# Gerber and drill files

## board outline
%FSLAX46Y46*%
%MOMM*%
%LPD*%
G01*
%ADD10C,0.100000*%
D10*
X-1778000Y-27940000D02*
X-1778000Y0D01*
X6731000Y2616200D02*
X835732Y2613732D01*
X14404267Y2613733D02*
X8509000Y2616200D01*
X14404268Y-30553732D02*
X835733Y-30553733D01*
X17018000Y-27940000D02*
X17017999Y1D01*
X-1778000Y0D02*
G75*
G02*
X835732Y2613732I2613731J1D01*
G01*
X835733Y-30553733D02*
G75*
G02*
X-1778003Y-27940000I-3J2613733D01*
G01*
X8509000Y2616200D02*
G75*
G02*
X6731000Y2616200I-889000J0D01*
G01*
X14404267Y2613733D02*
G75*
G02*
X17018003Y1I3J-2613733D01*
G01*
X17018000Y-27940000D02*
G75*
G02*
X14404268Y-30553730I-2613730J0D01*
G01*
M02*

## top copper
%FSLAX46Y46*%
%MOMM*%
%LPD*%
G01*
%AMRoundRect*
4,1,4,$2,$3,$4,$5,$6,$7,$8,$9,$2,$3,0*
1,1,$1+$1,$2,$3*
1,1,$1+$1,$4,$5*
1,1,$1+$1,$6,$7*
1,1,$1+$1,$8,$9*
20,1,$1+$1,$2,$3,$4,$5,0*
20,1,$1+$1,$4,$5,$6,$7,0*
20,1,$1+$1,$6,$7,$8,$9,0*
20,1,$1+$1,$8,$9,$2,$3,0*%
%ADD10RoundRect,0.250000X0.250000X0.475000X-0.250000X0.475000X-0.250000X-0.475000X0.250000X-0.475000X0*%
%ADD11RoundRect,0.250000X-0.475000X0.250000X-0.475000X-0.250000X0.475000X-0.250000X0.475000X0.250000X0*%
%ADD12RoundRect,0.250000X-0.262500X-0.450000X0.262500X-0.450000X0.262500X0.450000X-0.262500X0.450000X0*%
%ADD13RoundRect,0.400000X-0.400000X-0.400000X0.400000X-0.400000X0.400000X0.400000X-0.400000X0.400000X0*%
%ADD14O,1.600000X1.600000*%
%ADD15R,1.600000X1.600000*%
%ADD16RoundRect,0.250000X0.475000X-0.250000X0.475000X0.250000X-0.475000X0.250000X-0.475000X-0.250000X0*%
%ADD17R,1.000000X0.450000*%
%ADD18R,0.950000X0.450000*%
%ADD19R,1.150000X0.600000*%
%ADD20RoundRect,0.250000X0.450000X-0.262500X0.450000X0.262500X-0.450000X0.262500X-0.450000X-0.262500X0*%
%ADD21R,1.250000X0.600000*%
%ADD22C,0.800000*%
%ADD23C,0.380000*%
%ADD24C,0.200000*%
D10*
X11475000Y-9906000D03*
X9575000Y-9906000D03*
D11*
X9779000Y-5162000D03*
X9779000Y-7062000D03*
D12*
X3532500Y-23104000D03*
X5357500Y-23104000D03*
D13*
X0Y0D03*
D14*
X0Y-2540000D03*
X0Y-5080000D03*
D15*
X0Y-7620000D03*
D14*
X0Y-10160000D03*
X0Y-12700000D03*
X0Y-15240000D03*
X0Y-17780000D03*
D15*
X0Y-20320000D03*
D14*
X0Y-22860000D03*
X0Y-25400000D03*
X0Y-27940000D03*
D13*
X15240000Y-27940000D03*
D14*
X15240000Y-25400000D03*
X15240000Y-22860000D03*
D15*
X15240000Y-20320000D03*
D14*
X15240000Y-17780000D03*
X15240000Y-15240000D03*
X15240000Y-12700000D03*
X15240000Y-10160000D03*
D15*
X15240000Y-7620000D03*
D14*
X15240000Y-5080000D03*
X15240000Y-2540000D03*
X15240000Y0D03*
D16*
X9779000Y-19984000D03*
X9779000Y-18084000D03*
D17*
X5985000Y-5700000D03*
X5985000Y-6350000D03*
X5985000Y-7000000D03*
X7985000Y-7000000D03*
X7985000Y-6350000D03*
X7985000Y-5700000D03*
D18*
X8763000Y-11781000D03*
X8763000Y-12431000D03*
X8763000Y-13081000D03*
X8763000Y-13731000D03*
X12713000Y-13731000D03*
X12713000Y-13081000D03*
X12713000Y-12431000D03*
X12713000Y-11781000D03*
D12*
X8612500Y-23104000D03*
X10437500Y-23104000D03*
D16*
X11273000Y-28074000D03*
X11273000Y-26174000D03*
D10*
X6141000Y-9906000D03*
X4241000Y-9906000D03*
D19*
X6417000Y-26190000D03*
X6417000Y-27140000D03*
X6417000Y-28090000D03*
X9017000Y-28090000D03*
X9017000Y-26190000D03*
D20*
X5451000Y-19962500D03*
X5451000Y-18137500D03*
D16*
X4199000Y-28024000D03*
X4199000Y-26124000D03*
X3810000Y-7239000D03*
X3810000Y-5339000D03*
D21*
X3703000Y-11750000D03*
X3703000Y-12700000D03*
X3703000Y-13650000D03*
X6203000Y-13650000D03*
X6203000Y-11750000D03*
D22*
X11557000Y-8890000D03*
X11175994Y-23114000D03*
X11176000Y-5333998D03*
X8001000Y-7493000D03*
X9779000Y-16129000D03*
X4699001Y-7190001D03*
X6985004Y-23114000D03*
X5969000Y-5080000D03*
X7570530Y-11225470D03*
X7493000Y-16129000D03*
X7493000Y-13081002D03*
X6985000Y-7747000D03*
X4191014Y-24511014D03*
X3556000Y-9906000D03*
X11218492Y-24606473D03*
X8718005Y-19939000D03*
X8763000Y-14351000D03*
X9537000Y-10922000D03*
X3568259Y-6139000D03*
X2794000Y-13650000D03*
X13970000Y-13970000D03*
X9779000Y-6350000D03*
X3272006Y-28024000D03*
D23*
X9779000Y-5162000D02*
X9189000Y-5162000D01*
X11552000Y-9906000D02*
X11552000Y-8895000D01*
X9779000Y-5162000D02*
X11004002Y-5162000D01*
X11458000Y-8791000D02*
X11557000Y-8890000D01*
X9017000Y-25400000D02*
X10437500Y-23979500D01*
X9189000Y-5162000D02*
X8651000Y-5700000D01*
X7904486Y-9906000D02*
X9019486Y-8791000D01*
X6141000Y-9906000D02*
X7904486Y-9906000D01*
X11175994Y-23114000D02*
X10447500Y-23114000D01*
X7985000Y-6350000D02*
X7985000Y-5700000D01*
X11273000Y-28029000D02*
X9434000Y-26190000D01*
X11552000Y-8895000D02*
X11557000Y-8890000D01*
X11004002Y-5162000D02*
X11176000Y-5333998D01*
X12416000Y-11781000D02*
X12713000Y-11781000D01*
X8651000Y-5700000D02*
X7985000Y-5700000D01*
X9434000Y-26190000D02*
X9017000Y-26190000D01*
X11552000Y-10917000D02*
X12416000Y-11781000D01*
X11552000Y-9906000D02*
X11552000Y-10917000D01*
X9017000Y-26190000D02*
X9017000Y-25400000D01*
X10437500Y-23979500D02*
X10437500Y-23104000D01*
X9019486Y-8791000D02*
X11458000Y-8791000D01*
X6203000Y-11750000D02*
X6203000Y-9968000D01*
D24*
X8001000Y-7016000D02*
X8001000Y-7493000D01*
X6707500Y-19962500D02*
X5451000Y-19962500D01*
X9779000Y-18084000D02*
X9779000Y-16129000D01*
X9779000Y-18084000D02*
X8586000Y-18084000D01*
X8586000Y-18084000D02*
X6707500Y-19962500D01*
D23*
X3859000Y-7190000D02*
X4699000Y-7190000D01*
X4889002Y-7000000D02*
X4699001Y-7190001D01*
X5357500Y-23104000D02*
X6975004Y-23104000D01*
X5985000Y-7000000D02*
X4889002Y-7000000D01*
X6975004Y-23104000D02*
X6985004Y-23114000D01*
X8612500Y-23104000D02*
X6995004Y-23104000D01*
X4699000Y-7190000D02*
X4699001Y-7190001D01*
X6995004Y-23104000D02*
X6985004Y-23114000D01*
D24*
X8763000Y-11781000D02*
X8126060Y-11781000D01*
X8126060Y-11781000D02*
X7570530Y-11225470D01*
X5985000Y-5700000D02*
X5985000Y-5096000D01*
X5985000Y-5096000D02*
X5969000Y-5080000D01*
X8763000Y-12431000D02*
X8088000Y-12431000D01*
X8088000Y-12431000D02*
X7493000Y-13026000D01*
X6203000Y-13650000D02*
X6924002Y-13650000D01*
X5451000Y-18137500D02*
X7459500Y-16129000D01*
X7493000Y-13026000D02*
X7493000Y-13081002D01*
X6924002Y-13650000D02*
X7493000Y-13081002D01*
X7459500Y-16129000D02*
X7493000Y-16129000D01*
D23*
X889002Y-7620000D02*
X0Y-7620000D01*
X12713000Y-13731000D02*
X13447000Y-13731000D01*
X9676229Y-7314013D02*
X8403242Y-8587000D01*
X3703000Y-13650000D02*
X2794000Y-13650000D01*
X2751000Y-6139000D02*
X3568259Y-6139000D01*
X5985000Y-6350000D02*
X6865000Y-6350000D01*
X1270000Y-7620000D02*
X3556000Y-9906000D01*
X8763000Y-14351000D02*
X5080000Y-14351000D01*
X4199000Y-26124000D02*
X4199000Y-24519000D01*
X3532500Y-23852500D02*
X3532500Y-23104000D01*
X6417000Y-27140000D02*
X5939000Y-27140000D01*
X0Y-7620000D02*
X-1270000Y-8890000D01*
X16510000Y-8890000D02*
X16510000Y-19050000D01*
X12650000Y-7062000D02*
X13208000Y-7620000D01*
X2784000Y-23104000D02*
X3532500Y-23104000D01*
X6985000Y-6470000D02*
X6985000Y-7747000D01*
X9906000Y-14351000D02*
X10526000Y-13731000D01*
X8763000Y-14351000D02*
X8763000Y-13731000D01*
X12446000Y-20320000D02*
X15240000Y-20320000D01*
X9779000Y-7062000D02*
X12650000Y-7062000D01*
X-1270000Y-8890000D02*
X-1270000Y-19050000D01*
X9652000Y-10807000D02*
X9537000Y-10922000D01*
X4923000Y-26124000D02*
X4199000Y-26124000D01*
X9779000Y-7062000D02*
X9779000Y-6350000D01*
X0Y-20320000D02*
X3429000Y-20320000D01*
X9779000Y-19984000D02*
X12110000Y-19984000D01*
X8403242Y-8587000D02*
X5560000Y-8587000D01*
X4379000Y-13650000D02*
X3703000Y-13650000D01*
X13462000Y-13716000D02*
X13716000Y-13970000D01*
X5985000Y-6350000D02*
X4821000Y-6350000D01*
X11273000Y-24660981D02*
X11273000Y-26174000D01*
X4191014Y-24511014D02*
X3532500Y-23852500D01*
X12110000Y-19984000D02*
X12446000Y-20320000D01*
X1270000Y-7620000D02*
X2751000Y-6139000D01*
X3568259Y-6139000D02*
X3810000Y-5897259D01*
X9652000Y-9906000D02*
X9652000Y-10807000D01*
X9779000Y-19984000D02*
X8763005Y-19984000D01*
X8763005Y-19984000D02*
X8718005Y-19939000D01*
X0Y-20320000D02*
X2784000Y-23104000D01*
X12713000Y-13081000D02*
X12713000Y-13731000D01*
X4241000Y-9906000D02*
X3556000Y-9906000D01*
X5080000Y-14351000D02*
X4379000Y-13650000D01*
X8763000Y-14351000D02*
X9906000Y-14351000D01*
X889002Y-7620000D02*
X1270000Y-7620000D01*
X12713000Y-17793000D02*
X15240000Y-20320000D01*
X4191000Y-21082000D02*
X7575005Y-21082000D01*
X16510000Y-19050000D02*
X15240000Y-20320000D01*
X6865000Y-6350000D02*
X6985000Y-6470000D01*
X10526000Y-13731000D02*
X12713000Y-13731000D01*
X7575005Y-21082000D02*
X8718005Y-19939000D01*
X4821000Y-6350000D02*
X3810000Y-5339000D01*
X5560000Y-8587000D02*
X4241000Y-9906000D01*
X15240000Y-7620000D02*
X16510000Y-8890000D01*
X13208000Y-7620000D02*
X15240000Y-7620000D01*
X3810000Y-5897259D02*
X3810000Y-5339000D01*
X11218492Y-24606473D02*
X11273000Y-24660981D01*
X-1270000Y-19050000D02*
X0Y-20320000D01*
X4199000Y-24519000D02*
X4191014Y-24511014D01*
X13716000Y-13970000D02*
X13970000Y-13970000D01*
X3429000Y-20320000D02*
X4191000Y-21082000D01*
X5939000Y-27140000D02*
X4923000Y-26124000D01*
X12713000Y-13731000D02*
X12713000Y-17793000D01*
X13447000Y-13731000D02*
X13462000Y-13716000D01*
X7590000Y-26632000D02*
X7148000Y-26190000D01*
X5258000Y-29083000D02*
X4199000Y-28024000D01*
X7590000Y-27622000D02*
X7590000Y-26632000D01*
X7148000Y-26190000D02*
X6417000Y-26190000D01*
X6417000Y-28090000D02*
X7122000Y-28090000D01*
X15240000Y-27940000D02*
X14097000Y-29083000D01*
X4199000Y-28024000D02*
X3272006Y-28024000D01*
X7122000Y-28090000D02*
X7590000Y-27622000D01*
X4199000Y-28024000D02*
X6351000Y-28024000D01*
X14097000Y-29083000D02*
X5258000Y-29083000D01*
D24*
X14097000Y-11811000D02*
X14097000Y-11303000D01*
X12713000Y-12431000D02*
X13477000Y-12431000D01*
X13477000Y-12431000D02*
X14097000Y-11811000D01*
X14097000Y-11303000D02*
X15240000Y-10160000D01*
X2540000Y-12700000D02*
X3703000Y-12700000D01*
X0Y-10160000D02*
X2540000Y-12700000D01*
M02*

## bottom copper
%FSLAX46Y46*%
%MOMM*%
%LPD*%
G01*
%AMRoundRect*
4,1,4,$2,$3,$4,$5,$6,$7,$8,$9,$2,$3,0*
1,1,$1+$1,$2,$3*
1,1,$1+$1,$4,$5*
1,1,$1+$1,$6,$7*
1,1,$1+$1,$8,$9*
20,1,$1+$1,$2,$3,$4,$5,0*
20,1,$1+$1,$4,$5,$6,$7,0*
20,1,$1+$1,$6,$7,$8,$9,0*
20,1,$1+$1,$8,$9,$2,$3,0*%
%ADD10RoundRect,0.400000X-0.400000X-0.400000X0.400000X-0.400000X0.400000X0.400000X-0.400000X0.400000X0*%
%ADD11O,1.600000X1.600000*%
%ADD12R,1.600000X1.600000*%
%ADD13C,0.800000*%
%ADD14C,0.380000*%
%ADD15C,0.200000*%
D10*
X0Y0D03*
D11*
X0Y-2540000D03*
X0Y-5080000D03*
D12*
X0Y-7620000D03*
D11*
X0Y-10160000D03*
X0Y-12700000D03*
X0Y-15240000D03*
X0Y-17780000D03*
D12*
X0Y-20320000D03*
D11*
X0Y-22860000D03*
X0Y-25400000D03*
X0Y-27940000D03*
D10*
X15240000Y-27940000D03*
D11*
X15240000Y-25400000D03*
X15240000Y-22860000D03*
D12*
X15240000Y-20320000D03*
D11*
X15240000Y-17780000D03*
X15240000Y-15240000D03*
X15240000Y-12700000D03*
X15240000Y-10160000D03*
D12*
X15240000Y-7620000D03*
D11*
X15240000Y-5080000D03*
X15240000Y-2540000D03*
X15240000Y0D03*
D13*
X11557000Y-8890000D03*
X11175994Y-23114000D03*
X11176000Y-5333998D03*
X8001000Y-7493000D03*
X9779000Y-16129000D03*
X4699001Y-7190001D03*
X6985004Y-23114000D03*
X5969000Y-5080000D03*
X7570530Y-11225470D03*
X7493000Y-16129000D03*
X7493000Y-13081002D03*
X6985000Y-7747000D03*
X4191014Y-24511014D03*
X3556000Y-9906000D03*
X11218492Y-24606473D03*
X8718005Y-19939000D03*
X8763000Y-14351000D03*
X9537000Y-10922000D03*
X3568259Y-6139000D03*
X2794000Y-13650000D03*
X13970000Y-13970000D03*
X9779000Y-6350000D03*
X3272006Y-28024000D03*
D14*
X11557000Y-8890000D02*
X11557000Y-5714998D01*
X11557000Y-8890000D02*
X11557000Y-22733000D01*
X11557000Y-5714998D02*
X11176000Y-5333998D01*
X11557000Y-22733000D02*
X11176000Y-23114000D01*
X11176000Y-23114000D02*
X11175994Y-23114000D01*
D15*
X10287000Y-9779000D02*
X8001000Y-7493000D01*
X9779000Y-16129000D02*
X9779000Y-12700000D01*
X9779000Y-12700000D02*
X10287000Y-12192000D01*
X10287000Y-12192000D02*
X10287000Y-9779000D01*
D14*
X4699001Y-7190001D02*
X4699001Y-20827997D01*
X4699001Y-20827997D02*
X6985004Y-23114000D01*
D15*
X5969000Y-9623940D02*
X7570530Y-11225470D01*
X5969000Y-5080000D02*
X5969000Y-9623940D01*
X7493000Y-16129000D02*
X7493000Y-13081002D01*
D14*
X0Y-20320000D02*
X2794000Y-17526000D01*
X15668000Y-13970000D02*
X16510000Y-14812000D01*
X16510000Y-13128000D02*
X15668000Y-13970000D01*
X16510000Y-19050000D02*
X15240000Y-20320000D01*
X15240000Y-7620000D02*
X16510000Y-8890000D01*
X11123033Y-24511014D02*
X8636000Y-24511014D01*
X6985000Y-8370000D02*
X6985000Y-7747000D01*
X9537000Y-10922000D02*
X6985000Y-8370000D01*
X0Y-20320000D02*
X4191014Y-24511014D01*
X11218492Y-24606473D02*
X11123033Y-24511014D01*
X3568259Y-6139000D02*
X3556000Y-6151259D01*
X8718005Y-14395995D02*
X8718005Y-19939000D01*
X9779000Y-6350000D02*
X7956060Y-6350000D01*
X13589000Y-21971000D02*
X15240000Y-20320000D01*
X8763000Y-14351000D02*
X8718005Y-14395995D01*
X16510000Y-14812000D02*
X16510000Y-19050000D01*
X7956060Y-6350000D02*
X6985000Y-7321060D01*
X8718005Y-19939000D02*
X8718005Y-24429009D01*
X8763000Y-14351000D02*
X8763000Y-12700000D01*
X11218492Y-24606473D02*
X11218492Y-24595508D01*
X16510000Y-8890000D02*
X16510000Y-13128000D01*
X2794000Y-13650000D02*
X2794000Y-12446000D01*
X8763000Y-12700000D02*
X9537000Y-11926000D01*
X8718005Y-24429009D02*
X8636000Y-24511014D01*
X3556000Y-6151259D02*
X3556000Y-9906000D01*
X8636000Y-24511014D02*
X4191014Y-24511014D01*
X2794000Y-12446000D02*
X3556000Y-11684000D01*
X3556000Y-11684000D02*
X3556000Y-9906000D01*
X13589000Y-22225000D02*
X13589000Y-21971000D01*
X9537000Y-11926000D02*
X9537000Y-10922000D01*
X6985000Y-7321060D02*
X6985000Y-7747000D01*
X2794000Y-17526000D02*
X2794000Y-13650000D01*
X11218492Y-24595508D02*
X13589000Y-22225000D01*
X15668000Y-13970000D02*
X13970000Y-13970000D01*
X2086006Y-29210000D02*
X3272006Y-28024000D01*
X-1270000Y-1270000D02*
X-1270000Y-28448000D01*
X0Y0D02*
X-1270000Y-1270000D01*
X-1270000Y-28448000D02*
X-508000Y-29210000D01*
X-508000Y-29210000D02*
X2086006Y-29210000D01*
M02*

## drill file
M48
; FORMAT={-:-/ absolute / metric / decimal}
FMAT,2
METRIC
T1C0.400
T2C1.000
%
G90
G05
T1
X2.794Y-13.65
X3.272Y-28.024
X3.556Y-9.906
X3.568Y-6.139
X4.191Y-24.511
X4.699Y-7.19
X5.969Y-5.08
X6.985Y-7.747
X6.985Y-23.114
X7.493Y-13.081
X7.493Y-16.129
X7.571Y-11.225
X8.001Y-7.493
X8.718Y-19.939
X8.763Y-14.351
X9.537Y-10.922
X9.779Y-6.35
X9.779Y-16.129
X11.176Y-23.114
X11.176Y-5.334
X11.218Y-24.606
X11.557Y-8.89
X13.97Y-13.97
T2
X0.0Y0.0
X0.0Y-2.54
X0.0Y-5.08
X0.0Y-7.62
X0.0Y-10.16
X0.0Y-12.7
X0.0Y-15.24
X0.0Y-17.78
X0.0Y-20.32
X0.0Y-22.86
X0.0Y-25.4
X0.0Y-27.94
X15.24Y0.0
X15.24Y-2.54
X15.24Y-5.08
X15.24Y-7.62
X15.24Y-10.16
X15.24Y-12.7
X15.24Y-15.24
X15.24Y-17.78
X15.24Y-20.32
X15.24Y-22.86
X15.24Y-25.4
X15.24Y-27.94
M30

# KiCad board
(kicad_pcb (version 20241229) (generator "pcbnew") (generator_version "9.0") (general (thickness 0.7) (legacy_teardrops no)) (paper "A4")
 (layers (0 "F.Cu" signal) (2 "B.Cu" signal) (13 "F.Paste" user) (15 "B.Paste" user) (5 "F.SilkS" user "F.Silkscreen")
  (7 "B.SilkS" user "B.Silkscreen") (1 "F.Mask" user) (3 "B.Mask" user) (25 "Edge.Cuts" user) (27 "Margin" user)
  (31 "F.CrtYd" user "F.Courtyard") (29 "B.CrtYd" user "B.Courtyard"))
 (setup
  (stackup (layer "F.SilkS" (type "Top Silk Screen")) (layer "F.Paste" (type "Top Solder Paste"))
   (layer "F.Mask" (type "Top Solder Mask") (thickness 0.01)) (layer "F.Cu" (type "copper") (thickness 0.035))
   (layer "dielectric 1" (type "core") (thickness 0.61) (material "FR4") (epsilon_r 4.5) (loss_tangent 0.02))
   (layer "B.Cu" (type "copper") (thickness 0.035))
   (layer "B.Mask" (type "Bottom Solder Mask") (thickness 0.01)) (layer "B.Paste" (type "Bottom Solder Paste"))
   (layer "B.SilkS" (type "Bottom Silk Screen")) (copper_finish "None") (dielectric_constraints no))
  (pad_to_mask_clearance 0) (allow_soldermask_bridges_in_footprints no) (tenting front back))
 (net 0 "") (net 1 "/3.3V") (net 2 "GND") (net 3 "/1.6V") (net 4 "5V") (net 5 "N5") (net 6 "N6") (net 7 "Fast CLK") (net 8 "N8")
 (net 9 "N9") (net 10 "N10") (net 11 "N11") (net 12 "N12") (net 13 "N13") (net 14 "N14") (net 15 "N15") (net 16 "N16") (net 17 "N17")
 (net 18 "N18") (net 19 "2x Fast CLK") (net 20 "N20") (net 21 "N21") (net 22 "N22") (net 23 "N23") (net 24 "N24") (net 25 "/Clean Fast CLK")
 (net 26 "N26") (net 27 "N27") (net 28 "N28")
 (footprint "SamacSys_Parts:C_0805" (layer "F.Cu") (at 10.541 9.906 90)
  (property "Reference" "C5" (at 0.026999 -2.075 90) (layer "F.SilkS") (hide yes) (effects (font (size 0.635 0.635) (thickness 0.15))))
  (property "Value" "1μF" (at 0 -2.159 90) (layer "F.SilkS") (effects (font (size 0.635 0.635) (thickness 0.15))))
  (pad "1" smd roundrect (at 0 0.934 180) (size 1 1.45) (layers "F.Cu" "F.Mask" "F.Paste") (roundrect_rratio 0.25) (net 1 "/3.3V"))
  (pad "2" smd roundrect (at 0 -0.966 180) (size 1 1.45) (layers "F.Cu" "F.Mask" "F.Paste") (roundrect_rratio 0.25) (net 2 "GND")))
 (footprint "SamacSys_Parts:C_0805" (layer "F.Cu") (at 9.779 6.096 180)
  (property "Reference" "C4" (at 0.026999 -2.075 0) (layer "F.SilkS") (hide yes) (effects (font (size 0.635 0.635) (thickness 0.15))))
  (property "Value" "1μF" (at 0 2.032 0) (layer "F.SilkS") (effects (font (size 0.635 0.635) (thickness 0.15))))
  (pad "1" smd roundrect (at 0 0.934 270) (size 1 1.45) (layers "F.Cu" "F.Mask" "F.Paste") (roundrect_rratio 0.25) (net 1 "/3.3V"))
  (pad "2" smd roundrect (at 0 -0.966 270) (size 1 1.45) (layers "F.Cu" "F.Mask" "F.Paste") (roundrect_rratio 0.25) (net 2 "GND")))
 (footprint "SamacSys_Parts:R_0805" (layer "F.Cu") (at 4.445 23.114 -90)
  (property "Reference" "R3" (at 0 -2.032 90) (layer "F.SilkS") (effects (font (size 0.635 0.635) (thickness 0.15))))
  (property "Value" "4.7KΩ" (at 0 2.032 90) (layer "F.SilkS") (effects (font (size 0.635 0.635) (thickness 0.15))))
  (pad "1" smd roundrect (at -0.01 0.9125) (size 1.025 1.4) (layers "F.Cu" "F.Mask" "F.Paste") (roundrect_rratio 0.243902) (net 2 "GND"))
  (pad "2" smd roundrect (at -0.01 -0.9125) (size 1.025 1.4) (layers "F.Cu" "F.Mask" "F.Paste") (roundrect_rratio 0.243902) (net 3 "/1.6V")))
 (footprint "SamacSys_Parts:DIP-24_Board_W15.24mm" (layer "F.Cu") (at 0 0)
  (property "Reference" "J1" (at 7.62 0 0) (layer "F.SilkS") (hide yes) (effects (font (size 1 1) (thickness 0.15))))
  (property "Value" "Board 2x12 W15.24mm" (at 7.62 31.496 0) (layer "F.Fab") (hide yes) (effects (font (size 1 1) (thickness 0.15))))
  (fp_line (start -1.778 27.94) (end -1.778 0) (stroke (width 0.1) (type solid)) (layer "Edge.Cuts"))
  (fp_line (start 6.731 -2.6162) (end 0.835732 -2.613732) (stroke (width 0.1) (type solid)) (layer "Edge.Cuts"))
  (fp_line (start 14.404267 -2.613733) (end 8.509 -2.6162) (stroke (width 0.1) (type solid)) (layer "Edge.Cuts"))
  (fp_line (start 14.404268 30.553732) (end 0.835733 30.553733) (stroke (width 0.1) (type solid)) (layer "Edge.Cuts"))
  (fp_line (start 17.018 27.94) (end 17.017999 -0.000001) (stroke (width 0.1) (type solid)) (layer "Edge.Cuts"))
  (fp_arc (start -1.778 0) (mid -1.012456 -1.848188) (end 0.835732 -2.613732) (stroke (width 0.1) (type solid)) (layer "Edge.Cuts"))
  (fp_arc (start 0.835733 30.553733) (mid -1.012456 29.788189) (end -1.778 27.94) (stroke (width 0.1) (type solid)) (layer "Edge.Cuts"))
  (fp_arc (start 8.509 -2.6162) (mid 7.62 -1.7272) (end 6.731 -2.6162) (stroke (width 0.1) (type default)) (layer "Edge.Cuts"))
  (fp_arc (start 14.404267 -2.613733) (mid 16.252455 -1.848189) (end 17.017999 -0.000001) (stroke (width 0.1) (type solid))
   (layer "Edge.Cuts"))
  (fp_arc (start 17.018 27.94) (mid 16.252455 29.788187) (end 14.404268 30.553732) (stroke (width 0.1) (type solid)) (layer "Edge.Cuts"))
  (pad "1" thru_hole roundrect (at 0 0) (size 1.6 1.6) (drill 1) (layers "*.Cu" "*.Mask") (remove_unused_layers no) (roundrect_rratio 0.25)
   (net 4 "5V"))
  (pad "2" thru_hole oval (at 0 2.54) (size 1.6 1.6) (drill 1) (layers "*.Cu" "*.Mask") (remove_unused_layers no) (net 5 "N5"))
  (pad "3" thru_hole oval (at 0 5.08) (size 1.6 1.6) (drill 1) (layers "*.Cu" "*.Mask") (remove_unused_layers no) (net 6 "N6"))
  (pad "4" thru_hole rect (at 0 7.62) (size 1.6 1.6) (drill 1) (layers "*.Cu" "*.Mask") (remove_unused_layers no) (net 2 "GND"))
  (pad "5" thru_hole oval (at 0 10.16) (size 1.6 1.6) (drill 1) (layers "*.Cu" "*.Mask") (remove_unused_layers no) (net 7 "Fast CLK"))
  (pad "6" thru_hole oval (at 0 12.7) (size 1.6 1.6) (drill 1) (layers "*.Cu" "*.Mask") (remove_unused_layers no) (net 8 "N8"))
  (pad "7" thru_hole oval (at 0 15.24) (size 1.6 1.6) (drill 1) (layers "*.Cu" "*.Mask") (remove_unused_layers no) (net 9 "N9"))
  (pad "8" thru_hole oval (at 0 17.78) (size 1.6 1.6) (drill 1) (layers "*.Cu" "*.Mask") (remove_unused_layers no) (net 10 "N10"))
  (pad "9" thru_hole rect (at 0 20.32) (size 1.6 1.6) (drill 1) (layers "*.Cu" "*.Mask") (remove_unused_layers no) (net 2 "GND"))
  (pad "10" thru_hole oval (at 0 22.86) (size 1.6 1.6) (drill 1) (layers "*.Cu" "*.Mask") (remove_unused_layers no) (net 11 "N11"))
  (pad "11" thru_hole oval (at 0 25.4) (size 1.6 1.6) (drill 1) (layers "*.Cu" "*.Mask") (remove_unused_layers no) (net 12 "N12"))
  (pad "12" thru_hole oval (at 0 27.94) (size 1.6 1.6) (drill 1) (layers "*.Cu" "*.Mask") (remove_unused_layers no) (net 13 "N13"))
  (pad "13" thru_hole roundrect (at 15.24 27.94) (size 1.6 1.6) (drill 1) (layers "*.Cu" "*.Mask") (remove_unused_layers no)
   (roundrect_rratio 0.25) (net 4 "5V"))
  (pad "14" thru_hole oval (at 15.24 25.4) (size 1.6 1.6) (drill 1) (layers "*.Cu" "*.Mask") (remove_unused_layers no) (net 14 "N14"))
  (pad "15" thru_hole oval (at 15.24 22.86) (size 1.6 1.6) (drill 1) (layers "*.Cu" "*.Mask") (remove_unused_layers no) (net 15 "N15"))
  (pad "16" thru_hole rect (at 15.24 20.32) (size 1.6 1.6) (drill 1) (layers "*.Cu" "*.Mask") (remove_unused_layers no) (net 2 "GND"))
  (pad "17" thru_hole oval (at 15.24 17.78 180) (size 1.6 1.6) (drill 1) (layers "*.Cu" "*.Mask") (remove_unused_layers no) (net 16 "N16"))
  (pad "18" thru_hole oval (at 15.24 15.24 180) (size 1.6 1.6) (drill 1) (layers "*.Cu" "*.Mask") (remove_unused_layers no) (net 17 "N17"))
  (pad "19" thru_hole oval (at 15.24 12.7 180) (size 1.6 1.6) (drill 1) (layers "*.Cu" "*.Mask") (remove_unused_layers no) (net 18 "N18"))
  (pad "20" thru_hole oval (at 15.24 10.16 180) (size 1.6 1.6) (drill 1) (layers "*.Cu" "*.Mask") (remove_unused_layers no)
   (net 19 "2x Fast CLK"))
  (pad "21" thru_hole rect (at 15.24 7.62) (size 1.6 1.6) (drill 1) (layers "*.Cu" "*.Mask") (remove_unused_layers no) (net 2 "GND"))
  (pad "22" thru_hole oval (at 15.24 5.08) (size 1.6 1.6) (drill 1) (layers "*.Cu" "*.Mask") (remove_unused_layers no) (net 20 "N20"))
  (pad "23" thru_hole oval (at 15.24 2.54) (size 1.6 1.6) (drill 1) (layers "*.Cu" "*.Mask") (remove_unused_layers no) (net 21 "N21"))
  (pad "24" thru_hole oval (at 15.24 0) (size 1.6 1.6) (drill 1) (layers "*.Cu" "*.Mask") (remove_unused_layers no) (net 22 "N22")))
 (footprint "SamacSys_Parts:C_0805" (layer "F.Cu") (at 9.779 19.05)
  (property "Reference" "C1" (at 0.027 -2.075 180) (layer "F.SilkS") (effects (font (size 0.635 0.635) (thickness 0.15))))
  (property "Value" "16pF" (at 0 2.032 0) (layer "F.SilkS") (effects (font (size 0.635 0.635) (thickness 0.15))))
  (pad "1" smd roundrect (at 0 0.934 90) (size 1 1.45) (layers "F.Cu" "F.Mask" "F.Paste") (roundrect_rratio 0.25) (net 2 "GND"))
  (pad "2" smd roundrect (at 0 -0.966 90) (size 1 1.45) (layers "F.Cu" "F.Mask" "F.Paste") (roundrect_rratio 0.25) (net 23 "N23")))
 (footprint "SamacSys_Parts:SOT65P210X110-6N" (layer "F.Cu") (at 6.985 6.35)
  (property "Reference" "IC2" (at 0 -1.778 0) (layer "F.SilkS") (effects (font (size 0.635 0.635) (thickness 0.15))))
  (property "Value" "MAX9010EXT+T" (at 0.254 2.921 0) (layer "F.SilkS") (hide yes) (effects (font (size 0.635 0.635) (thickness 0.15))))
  (pad "1" smd rect (at -1 -0.65 90) (size 0.45 1) (layers "F.Cu" "F.Mask" "F.Paste") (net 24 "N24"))
  (pad "2" smd rect (at -1 0 90) (size 0.45 1) (layers "F.Cu" "F.Mask" "F.Paste") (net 2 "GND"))
  (pad "3" smd rect (at -1 0.65 90) (size 0.45 1) (layers "F.Cu" "F.Mask" "F.Paste") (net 3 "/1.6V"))
  (pad "4" smd rect (at 1 0.65 90) (size 0.45 1) (layers "F.Cu" "F.Mask" "F.Paste") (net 23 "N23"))
  (pad "5" smd rect (at 1 0 90) (size 0.45 1) (layers "F.Cu" "F.Mask" "F.Paste") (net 1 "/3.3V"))
  (pad "6" smd rect (at 1 -0.65 90) (size 0.45 1) (layers "F.Cu" "F.Mask" "F.Paste") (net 1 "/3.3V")))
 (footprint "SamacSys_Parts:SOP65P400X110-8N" (layer "F.Cu") (at 10.738 12.756)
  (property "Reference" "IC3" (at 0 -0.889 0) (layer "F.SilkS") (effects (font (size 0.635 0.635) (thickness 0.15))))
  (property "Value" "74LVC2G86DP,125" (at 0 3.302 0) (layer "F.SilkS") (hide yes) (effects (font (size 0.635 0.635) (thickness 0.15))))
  (pad "1" smd rect (at -1.975 -0.975 90) (size 0.45 0.95) (layers "F.Cu" "F.Mask" "F.Paste") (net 24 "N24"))
  (pad "2" smd rect (at -1.975 -0.325 90) (size 0.45 0.95) (layers "F.Cu" "F.Mask" "F.Paste") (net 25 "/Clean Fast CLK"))
  (pad "3" smd rect (at -1.975 0.325 90) (size 0.45 0.95) (layers "F.Cu" "F.Mask" "F.Paste") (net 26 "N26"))
  (pad "4" smd rect (at -1.975 0.975 90) (size 0.45 0.95) (layers "F.Cu" "F.Mask" "F.Paste") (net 2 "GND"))
  (pad "5" smd rect (at 1.975 0.975 90) (size 0.45 0.95) (layers "F.Cu" "F.Mask" "F.Paste") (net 2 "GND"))
  (pad "6" smd rect (at 1.975 0.325 90) (size 0.45 0.95) (layers "F.Cu" "F.Mask" "F.Paste") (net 2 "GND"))
  (pad "7" smd rect (at 1.975 -0.325 90) (size 0.45 0.95) (layers "F.Cu" "F.Mask" "F.Paste") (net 19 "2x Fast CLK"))
  (pad "8" smd rect (at 1.975 -0.975 90) (size 0.45 0.95) (layers "F.Cu" "F.Mask" "F.Paste") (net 1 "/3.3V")))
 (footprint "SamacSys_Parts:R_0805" (layer "F.Cu") (at 9.525 23.114 -90)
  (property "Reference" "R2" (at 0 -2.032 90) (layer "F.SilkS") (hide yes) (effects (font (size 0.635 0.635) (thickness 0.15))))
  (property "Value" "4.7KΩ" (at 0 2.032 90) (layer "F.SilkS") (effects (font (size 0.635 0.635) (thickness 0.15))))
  (pad "1" smd roundrect (at -0.01 0.9125) (size 1.025 1.4) (layers "F.Cu" "F.Mask" "F.Paste") (roundrect_rratio 0.243902) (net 3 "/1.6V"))
  (pad "2" smd roundrect (at -0.01 -0.9125) (size 1.025 1.4) (layers "F.Cu" "F.Mask" "F.Paste") (roundrect_rratio 0.243902) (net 1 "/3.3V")))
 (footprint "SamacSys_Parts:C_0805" (layer "F.Cu") (at 11.273 27.14)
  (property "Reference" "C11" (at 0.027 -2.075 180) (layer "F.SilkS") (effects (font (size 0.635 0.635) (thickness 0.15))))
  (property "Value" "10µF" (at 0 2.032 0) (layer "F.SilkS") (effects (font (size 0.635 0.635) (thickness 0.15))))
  (pad "1" smd roundrect (at 0 0.934 90) (size 1 1.45) (layers "F.Cu" "F.Mask" "F.Paste") (roundrect_rratio 0.25) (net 1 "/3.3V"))
  (pad "2" smd roundrect (at 0 -0.966 90) (size 1 1.45) (layers "F.Cu" "F.Mask" "F.Paste") (roundrect_rratio 0.25) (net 2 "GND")))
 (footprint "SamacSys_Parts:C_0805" (layer "F.Cu") (at 5.207 9.906 90)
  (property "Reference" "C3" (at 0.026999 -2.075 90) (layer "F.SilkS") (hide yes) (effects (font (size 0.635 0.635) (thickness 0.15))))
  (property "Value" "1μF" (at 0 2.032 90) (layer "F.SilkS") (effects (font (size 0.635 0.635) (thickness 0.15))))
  (pad "1" smd roundrect (at 0 0.934 180) (size 1 1.45) (layers "F.Cu" "F.Mask" "F.Paste") (roundrect_rratio 0.25) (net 1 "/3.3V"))
  (pad "2" smd roundrect (at 0 -0.966 180) (size 1 1.45) (layers "F.Cu" "F.Mask" "F.Paste") (roundrect_rratio 0.25) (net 2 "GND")))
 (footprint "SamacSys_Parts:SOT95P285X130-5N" (layer "F.Cu") (at 7.717 27.14)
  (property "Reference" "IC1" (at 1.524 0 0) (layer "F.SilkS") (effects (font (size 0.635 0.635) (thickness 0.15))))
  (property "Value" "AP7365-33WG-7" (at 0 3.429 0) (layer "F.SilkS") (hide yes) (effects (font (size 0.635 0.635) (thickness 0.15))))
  (pad "1" smd rect (at -1.3 -0.95 90) (size 0.6 1.15) (layers "F.Cu" "F.Mask" "F.Paste") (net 4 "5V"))
  (pad "2" smd rect (at -1.3 0 90) (size 0.6 1.15) (layers "F.Cu" "F.Mask" "F.Paste") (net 2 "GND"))
  (pad "3" smd rect (at -1.3 0.95 90) (size 0.6 1.15) (layers "F.Cu" "F.Mask" "F.Paste") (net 4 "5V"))
  (pad "4" smd rect (at 1.3 0.95 90) (size 0.6 1.15) (layers "F.Cu" "F.Mask" "F.Paste") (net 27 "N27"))
  (pad "5" smd rect (at 1.3 -0.95 90) (size 0.6 1.15) (layers "F.Cu" "F.Mask" "F.Paste") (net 1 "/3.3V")))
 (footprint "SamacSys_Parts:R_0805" (layer "F.Cu") (at 5.461 19.05)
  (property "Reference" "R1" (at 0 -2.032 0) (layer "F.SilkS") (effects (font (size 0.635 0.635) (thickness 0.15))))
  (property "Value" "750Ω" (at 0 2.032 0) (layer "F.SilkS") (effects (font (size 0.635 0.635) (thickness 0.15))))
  (pad "1" smd roundrect (at -0.01 0.9125 90) (size 1.025 1.4) (layers "F.Cu" "F.Mask" "F.Paste") (roundrect_rratio 0.243902) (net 23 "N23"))
  (pad "2" smd roundrect (at -0.01 -0.9125 90) (size 1.025 1.4) (layers "F.Cu" "F.Mask" "F.Paste") (roundrect_rratio 0.243902)
   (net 25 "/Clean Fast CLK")))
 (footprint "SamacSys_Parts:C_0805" (layer "F.Cu") (at 4.199 27.09)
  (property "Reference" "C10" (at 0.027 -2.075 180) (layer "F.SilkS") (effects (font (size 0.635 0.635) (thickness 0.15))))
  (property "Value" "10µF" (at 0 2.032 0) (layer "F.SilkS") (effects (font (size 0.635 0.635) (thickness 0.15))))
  (pad "1" smd roundrect (at 0 0.934 90) (size 1 1.45) (layers "F.Cu" "F.Mask" "F.Paste") (roundrect_rratio 0.25) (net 4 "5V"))
  (pad "2" smd roundrect (at 0 -0.966 90) (size 1 1.45) (layers "F.Cu" "F.Mask" "F.Paste") (roundrect_rratio 0.25) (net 2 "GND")))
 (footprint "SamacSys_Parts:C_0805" (layer "F.Cu") (at 3.81 6.305)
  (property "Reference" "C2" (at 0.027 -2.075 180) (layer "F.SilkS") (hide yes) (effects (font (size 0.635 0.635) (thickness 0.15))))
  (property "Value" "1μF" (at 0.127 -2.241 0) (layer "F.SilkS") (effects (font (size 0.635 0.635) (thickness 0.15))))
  (pad "1" smd roundrect (at 0 0.934 90) (size 1 1.45) (layers "F.Cu" "F.Mask" "F.Paste") (roundrect_rratio 0.25) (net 3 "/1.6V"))
  (pad "2" smd roundrect (at 0 -0.966 90) (size 1 1.45) (layers "F.Cu" "F.Mask" "F.Paste") (roundrect_rratio 0.25) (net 2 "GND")))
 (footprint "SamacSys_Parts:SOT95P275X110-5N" (layer "F.Cu") (at 4.953 12.7)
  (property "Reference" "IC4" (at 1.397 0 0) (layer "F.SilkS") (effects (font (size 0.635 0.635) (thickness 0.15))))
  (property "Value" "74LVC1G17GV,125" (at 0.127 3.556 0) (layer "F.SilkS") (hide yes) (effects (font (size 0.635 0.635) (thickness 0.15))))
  (pad "1" smd rect (at -1.25 -0.95 90) (size 0.6 1.25) (layers "F.Cu" "F.Mask" "F.Paste") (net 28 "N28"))
  (pad "2" smd rect (at -1.25 0 90) (size 0.6 1.25) (layers "F.Cu" "F.Mask" "F.Paste") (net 7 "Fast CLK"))
  (pad "3" smd rect (at -1.25 0.95 90) (size 0.6 1.25) (layers "F.Cu" "F.Mask" "F.Paste") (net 2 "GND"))
  (pad "4" smd rect (at 1.25 0.95 90) (size 0.6 1.25) (layers "F.Cu" "F.Mask" "F.Paste") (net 25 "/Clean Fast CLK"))
  (pad "5" smd rect (at 1.25 -0.95 90) (size 0.6 1.25) (layers "F.Cu" "F.Mask" "F.Paste") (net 1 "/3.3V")))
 (segment (start 9.779 5.162) (end 9.189 5.162) (width 0.38) (layer "F.Cu") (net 1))
 (segment (start 11.552 9.906) (end 11.552 8.895) (width 0.38) (layer "F.Cu") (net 1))
 (segment (start 9.779 5.162) (end 11.004002 5.162) (width 0.38) (layer "F.Cu") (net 1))
 (segment (start 11.458 8.791) (end 11.557 8.89) (width 0.38) (layer "F.Cu") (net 1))
 (segment (start 9.017 25.4) (end 10.4375 23.9795) (width 0.38) (layer "F.Cu") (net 1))
 (segment (start 9.189 5.162) (end 8.651 5.7) (width 0.38) (layer "F.Cu") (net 1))
 (segment (start 7.904486 9.906) (end 9.019486 8.791) (width 0.38) (layer "F.Cu") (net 1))
 (segment (start 6.141 9.906) (end 7.904486 9.906) (width 0.38) (layer "F.Cu") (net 1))
 (segment (start 11.175994 23.114) (end 10.4475 23.114) (width 0.38) (layer "F.Cu") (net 1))
 (segment (start 7.985 6.35) (end 7.985 5.7) (width 0.38) (layer "F.Cu") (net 1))
 (segment (start 11.273 28.029) (end 9.434 26.19) (width 0.38) (layer "F.Cu") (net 1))
 (segment (start 11.552 8.895) (end 11.557 8.89) (width 0.38) (layer "F.Cu") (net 1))
 (segment (start 11.004002 5.162) (end 11.176 5.333998) (width 0.38) (layer "F.Cu") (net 1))
 (segment (start 12.416 11.781) (end 12.713 11.781) (width 0.38) (layer "F.Cu") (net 1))
 (segment (start 8.651 5.7) (end 7.985 5.7) (width 0.38) (layer "F.Cu") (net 1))
 (segment (start 9.434 26.19) (end 9.017 26.19) (width 0.38) (layer "F.Cu") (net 1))
 (segment (start 11.552 10.917) (end 12.416 11.781) (width 0.38) (layer "F.Cu") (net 1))
 (segment (start 11.552 9.906) (end 11.552 10.917) (width 0.38) (layer "F.Cu") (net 1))
 (segment (start 9.017 26.19) (end 9.017 25.4) (width 0.38) (layer "F.Cu") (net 1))
 (segment (start 10.4375 23.9795) (end 10.4375 23.104) (width 0.38) (layer "F.Cu") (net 1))
 (segment (start 9.019486 8.791) (end 11.458 8.791) (width 0.38) (layer "F.Cu") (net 1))
 (segment (start 6.203 11.75) (end 6.203 9.968) (width 0.38) (layer "F.Cu") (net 1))
 (via (at 11.557 8.89) (size 0.8) (drill 0.4) (layers "F.Cu" "B.Cu") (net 1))
 (via (at 11.175994 23.114) (size 0.8) (drill 0.4) (layers "F.Cu" "B.Cu") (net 1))
 (via (at 11.176 5.333998) (size 0.8) (drill 0.4) (layers "F.Cu" "B.Cu") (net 1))
 (segment (start 11.557 8.89) (end 11.557 5.714998) (width 0.38) (layer "B.Cu") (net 1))
 (segment (start 11.557 8.89) (end 11.557 22.733) (width 0.38) (layer "B.Cu") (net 1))
 (segment (start 11.557 5.714998) (end 11.176 5.333998) (width 0.38) (layer "B.Cu") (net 1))
 (segment (start 11.557 22.733) (end 11.176 23.114) (width 0.38) (layer "B.Cu") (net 1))
 (segment (start 11.176 23.114) (end 11.175994 23.114) (width 0.38) (layer "B.Cu") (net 1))
 (segment (start 8.001 7.016) (end 8.001 7.493) (width 0.2) (layer "F.Cu") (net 23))
 (segment (start 6.7075 19.9625) (end 5.451 19.9625) (width 0.2) (layer "F.Cu") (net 23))
 (segment (start 9.779 18.084) (end 9.779 16.129) (width 0.2) (layer "F.Cu") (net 23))
 (segment (start 9.779 18.084) (end 8.586 18.084) (width 0.2) (layer "F.Cu") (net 23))
 (segment (start 8.586 18.084) (end 6.7075 19.9625) (width 0.2) (layer "F.Cu") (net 23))
 (via (at 8.001 7.493) (size 0.8) (drill 0.4) (layers "F.Cu" "B.Cu") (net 23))
 (via (at 9.779 16.129) (size 0.8) (drill 0.4) (layers "F.Cu" "B.Cu") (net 23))
 (segment (start 10.287 9.779) (end 8.001 7.493) (width 0.2) (layer "B.Cu") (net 23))
 (segment (start 9.779 16.129) (end 9.779 12.7) (width 0.2) (layer "B.Cu") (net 23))
 (segment (start 9.779 12.7) (end 10.287 12.192) (width 0.2) (layer "B.Cu") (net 23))
 (segment (start 10.287 12.192) (end 10.287 9.779) (width 0.2) (layer "B.Cu") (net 23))
 (segment (start 3.859 7.19) (end 4.699 7.19) (width 0.38) (layer "F.Cu") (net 3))
 (segment (start 4.889002 7) (end 4.699001 7.190001) (width 0.38) (layer "F.Cu") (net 3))
 (segment (start 5.3575 23.104) (end 6.975004 23.104) (width 0.38) (layer "F.Cu") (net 3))
 (segment (start 5.985 7) (end 4.889002 7) (width 0.38) (layer "F.Cu") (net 3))
 (segment (start 6.975004 23.104) (end 6.985004 23.114) (width 0.38) (layer "F.Cu") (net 3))
 (segment (start 8.6125 23.104) (end 6.995004 23.104) (width 0.38) (layer "F.Cu") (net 3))
 (segment (start 4.699 7.19) (end 4.699001 7.190001) (width 0.38) (layer "F.Cu") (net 3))
 (segment (start 6.995004 23.104) (end 6.985004 23.114) (width 0.38) (layer "F.Cu") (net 3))
 (via (at 4.699001 7.190001) (size 0.8) (drill 0.4) (layers "F.Cu" "B.Cu") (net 3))
 (via (at 6.985004 23.114) (size 0.8) (drill 0.4) (layers "F.Cu" "B.Cu") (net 3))
 (segment (start 4.699001 7.190001) (end 4.699001 20.827997) (width 0.38) (layer "B.Cu") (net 3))
 (segment (start 4.699001 20.827997) (end 6.985004 23.114) (width 0.38) (layer "B.Cu") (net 3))
 (segment (start 8.763 11.781) (end 8.12606 11.781) (width 0.2) (layer "F.Cu") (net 24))
 (segment (start 8.12606 11.781) (end 7.57053 11.22547) (width 0.2) (layer "F.Cu") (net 24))
 (segment (start 5.985 5.7) (end 5.985 5.096) (width 0.2) (layer "F.Cu") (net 24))
 (segment (start 5.985 5.096) (end 5.969 5.08) (width 0.2) (layer "F.Cu") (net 24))
 (via (at 5.969 5.08) (size 0.8) (drill 0.4) (layers "F.Cu" "B.Cu") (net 24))
 (via (at 7.57053 11.22547) (size 0.8) (drill 0.4) (layers "F.Cu" "B.Cu") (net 24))
 (segment (start 5.969 9.62394) (end 7.57053 11.22547) (width 0.2) (layer "B.Cu") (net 24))
 (segment (start 5.969 5.08) (end 5.969 9.62394) (width 0.2) (layer "B.Cu") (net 24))
 (segment (start 8.763 12.431) (end 8.088 12.431) (width 0.2) (layer "F.Cu") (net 25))
 (segment (start 8.088 12.431) (end 7.493 13.026) (width 0.2) (layer "F.Cu") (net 25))
 (segment (start 6.203 13.65) (end 6.924002 13.65) (width 0.2) (layer "F.Cu") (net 25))
 (segment (start 5.451 18.1375) (end 7.4595 16.129) (width 0.2) (layer "F.Cu") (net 25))
 (segment (start 7.493 13.026) (end 7.493 13.081002) (width 0.2) (layer "F.Cu") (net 25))
 (segment (start 6.924002 13.65) (end 7.493 13.081002) (width 0.2) (layer "F.Cu") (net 25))
 (segment (start 7.4595 16.129) (end 7.493 16.129) (width 0.2) (layer "F.Cu") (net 25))
 (via (at 7.493 16.129) (size 0.8) (drill 0.4) (layers "F.Cu" "B.Cu") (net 25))
 (via (at 7.493 13.081002) (size 0.8) (drill 0.4) (layers "F.Cu" "B.Cu") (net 25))
 (segment (start 7.493 16.129) (end 7.493 13.081002) (width 0.2) (layer "B.Cu") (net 25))
 (segment (start 0.889002 7.62) (end 0 7.62) (width 0.38) (layer "F.Cu") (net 2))
 (segment (start 12.713 13.731) (end 13.447 13.731) (width 0.38) (layer "F.Cu") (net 2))
 (segment (start 9.676229 7.314013) (end 8.403242 8.587) (width 0.38) (layer "F.Cu") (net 2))
 (segment (start 3.703 13.65) (end 2.794 13.65) (width 0.38) (layer "F.Cu") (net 2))
 (segment (start 2.751 6.139) (end 3.568259 6.139) (width 0.38) (layer "F.Cu") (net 2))
 (segment (start 5.985 6.35) (end 6.865 6.35) (width 0.38) (layer "F.Cu") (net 2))
 (segment (start 1.27 7.62) (end 3.556 9.906) (width 0.38) (layer "F.Cu") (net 2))
 (segment (start 8.763 14.351) (end 5.08 14.351) (width 0.38) (layer "F.Cu") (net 2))
 (segment (start 4.199 26.124) (end 4.199 24.519) (width 0.38) (layer "F.Cu") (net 2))
 (segment (start 3.5325 23.8525) (end 3.5325 23.104) (width 0.38) (layer "F.Cu") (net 2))
 (segment (start 6.417 27.14) (end 5.939 27.14) (width 0.38) (layer "F.Cu") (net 2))
 (segment (start 0 7.62) (end -1.27 8.89) (width 0.38) (layer "F.Cu") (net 2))
 (segment (start 16.51 8.89) (end 16.51 19.05) (width 0.38) (layer "F.Cu") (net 2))
 (segment (start 12.65 7.062) (end 13.208 7.62) (width 0.38) (layer "F.Cu") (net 2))
 (segment (start 2.784 23.104) (end 3.5325 23.104) (width 0.38) (layer "F.Cu") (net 2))
 (segment (start 6.985 6.47) (end 6.985 7.747) (width 0.38) (layer "F.Cu") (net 2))
 (segment (start 9.906 14.351) (end 10.526 13.731) (width 0.38) (layer "F.Cu") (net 2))
 (segment (start 8.763 14.351) (end 8.763 13.731) (width 0.38) (layer "F.Cu") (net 2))
 (segment (start 12.446 20.32) (end 15.24 20.32) (width 0.38) (layer "F.Cu") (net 2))
 (segment (start 9.779 7.062) (end 12.65 7.062) (width 0.38) (layer "F.Cu") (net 2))
 (segment (start -1.27 8.89) (end -1.27 19.05) (width 0.38) (layer "F.Cu") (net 2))
 (segment (start 9.652 10.807) (end 9.537 10.922) (width 0.38) (layer "F.Cu") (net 2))
 (segment (start 4.923 26.124) (end 4.199 26.124) (width 0.38) (layer "F.Cu") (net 2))
 (segment (start 9.779 7.062) (end 9.779 6.35) (width 0.38) (layer "F.Cu") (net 2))
 (segment (start 0 20.32) (end 3.429 20.32) (width 0.38) (layer "F.Cu") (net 2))
 (segment (start 9.779 19.984) (end 12.11 19.984) (width 0.38) (layer "F.Cu") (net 2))
 (segment (start 8.403242 8.587) (end 5.56 8.587) (width 0.38) (layer "F.Cu") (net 2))
 (segment (start 4.379 13.65) (end 3.703 13.65) (width 0.38) (layer "F.Cu") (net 2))
 (segment (start 13.462 13.716) (end 13.716 13.97) (width 0.38) (layer "F.Cu") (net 2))
 (segment (start 5.985 6.35) (end 4.821 6.35) (width 0.38) (layer "F.Cu") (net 2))
 (segment (start 11.273 24.660981) (end 11.273 26.174) (width 0.38) (layer "F.Cu") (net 2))
 (segment (start 4.191014 24.511014) (end 3.5325 23.8525) (width 0.38) (layer "F.Cu") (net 2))
 (segment (start 12.11 19.984) (end 12.446 20.32) (width 0.38) (layer "F.Cu") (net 2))
 (segment (start 1.27 7.62) (end 2.751 6.139) (width 0.38) (layer "F.Cu") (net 2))
 (segment (start 3.568259 6.139) (end 3.81 5.897259) (width 0.38) (layer "F.Cu") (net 2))
 (segment (start 9.652 9.906) (end 9.652 10.807) (width 0.38) (layer "F.Cu") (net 2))
 (segment (start 9.779 19.984) (end 8.763005 19.984) (width 0.38) (layer "F.Cu") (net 2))
 (segment (start 8.763005 19.984) (end 8.718005 19.939) (width 0.38) (layer "F.Cu") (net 2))
 (segment (start 0 20.32) (end 2.784 23.104) (width 0.38) (layer "F.Cu") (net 2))
 (segment (start 12.713 13.081) (end 12.713 13.731) (width 0.38) (layer "F.Cu") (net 2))
 (segment (start 4.241 9.906) (end 3.556 9.906) (width 0.38) (layer "F.Cu") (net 2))
 (segment (start 5.08 14.351) (end 4.379 13.65) (width 0.38) (layer "F.Cu") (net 2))
 (segment (start 8.763 14.351) (end 9.906 14.351) (width 0.38) (layer "F.Cu") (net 2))
 (segment (start 0.889002 7.62) (end 1.27 7.62) (width 0.38) (layer "F.Cu") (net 2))
 (segment (start 12.713 17.793) (end 15.24 20.32) (width 0.38) (layer "F.Cu") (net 2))
 (segment (start 4.191 21.082) (end 7.575005 21.082) (width 0.38) (layer "F.Cu") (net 2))
 (segment (start 16.51 19.05) (end 15.24 20.32) (width 0.38) (layer "F.Cu") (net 2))
 (segment (start 6.865 6.35) (end 6.985 6.47) (width 0.38) (layer "F.Cu") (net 2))
 (segment (start 10.526 13.731) (end 12.713 13.731) (width 0.38) (layer "F.Cu") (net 2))
 (segment (start 7.575005 21.082) (end 8.718005 19.939) (width 0.38) (layer "F.Cu") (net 2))
 (segment (start 4.821 6.35) (end 3.81 5.339) (width 0.38) (layer "F.Cu") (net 2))
 (segment (start 5.56 8.587) (end 4.241 9.906) (width 0.38) (layer "F.Cu") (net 2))
 (segment (start 15.24 7.62) (end 16.51 8.89) (width 0.38) (layer "F.Cu") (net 2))
 (segment (start 13.208 7.62) (end 15.24 7.62) (width 0.38) (layer "F.Cu") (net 2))
 (segment (start 3.81 5.897259) (end 3.81 5.339) (width 0.38) (layer "F.Cu") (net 2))
 (segment (start 11.218492 24.606473) (end 11.273 24.660981) (width 0.38) (layer "F.Cu") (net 2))
 (segment (start -1.27 19.05) (end 0 20.32) (width 0.38) (layer "F.Cu") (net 2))
 (segment (start 4.199 24.519) (end 4.191014 24.511014) (width 0.38) (layer "F.Cu") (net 2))
 (segment (start 13.716 13.97) (end 13.97 13.97) (width 0.38) (layer "F.Cu") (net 2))
 (segment (start 3.429 20.32) (end 4.191 21.082) (width 0.38) (layer "F.Cu") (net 2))
 (segment (start 5.939 27.14) (end 4.923 26.124) (width 0.38) (layer "F.Cu") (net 2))
 (segment (start 12.713 13.731) (end 12.713 17.793) (width 0.38) (layer "F.Cu") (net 2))
 (segment (start 13.447 13.731) (end 13.462 13.716) (width 0.38) (layer "F.Cu") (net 2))
 (via (at 6.985 7.747) (size 0.8) (drill 0.4) (layers "F.Cu" "B.Cu") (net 2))
 (via (at 4.191014 24.511014) (size 0.8) (drill 0.4) (layers "F.Cu" "B.Cu") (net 2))
 (via (at 3.556 9.906) (size 0.8) (drill 0.4) (layers "F.Cu" "B.Cu") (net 2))
 (via (at 11.218492 24.606473) (size 0.8) (drill 0.4) (layers "F.Cu" "B.Cu") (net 2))
 (via (at 8.718005 19.939) (size 0.8) (drill 0.4) (layers "F.Cu" "B.Cu") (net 2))
 (via (at 8.763 14.351) (size 0.8) (drill 0.4) (layers "F.Cu" "B.Cu") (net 2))
 (via (at 9.537 10.922) (size 0.8) (drill 0.4) (layers "F.Cu" "B.Cu") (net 2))
 (via (at 3.568259 6.139) (size 0.8) (drill 0.4) (layers "F.Cu" "B.Cu") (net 2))
 (via (at 2.794 13.65) (size 0.8) (drill 0.4) (layers "F.Cu" "B.Cu") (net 2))
 (via (at 13.97 13.97) (size 0.8) (drill 0.4) (layers "F.Cu" "B.Cu") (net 2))
 (via (at 9.779 6.35) (size 0.8) (drill 0.4) (layers "F.Cu" "B.Cu") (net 2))
 (segment (start 0 20.32) (end 2.794 17.526) (width 0.38) (layer "B.Cu") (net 2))
 (segment (start 15.668 13.97) (end 16.51 14.812) (width 0.38) (layer "B.Cu") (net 2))
 (segment (start 16.51 13.128) (end 15.668 13.97) (width 0.38) (layer "B.Cu") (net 2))
 (segment (start 16.51 19.05) (end 15.24 20.32) (width 0.38) (layer "B.Cu") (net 2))
 (segment (start 15.24 7.62) (end 16.51 8.89) (width 0.38) (layer "B.Cu") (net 2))
 (segment (start 11.123033 24.511014) (end 8.636 24.511014) (width 0.38) (layer "B.Cu") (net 2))
 (segment (start 6.985 8.37) (end 6.985 7.747) (width 0.38) (layer "B.Cu") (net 2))
 (segment (start 9.537 10.922) (end 6.985 8.37) (width 0.38) (layer "B.Cu") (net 2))
 (segment (start 0 20.32) (end 4.191014 24.511014) (width 0.38) (layer "B.Cu") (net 2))
 (segment (start 11.218492 24.606473) (end 11.123033 24.511014) (width 0.38) (layer "B.Cu") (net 2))
 (segment (start 3.568259 6.139) (end 3.556 6.151259) (width 0.38) (layer "B.Cu") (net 2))
 (segment (start 8.718005 14.395995) (end 8.718005 19.939) (width 0.38) (layer "B.Cu") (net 2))
 (segment (start 9.779 6.35) (end 7.95606 6.35) (width 0.38) (layer "B.Cu") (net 2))
 (segment (start 13.589 21.971) (end 15.24 20.32) (width 0.38) (layer "B.Cu") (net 2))
 (segment (start 8.763 14.351) (end 8.718005 14.395995) (width 0.38) (layer "B.Cu") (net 2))
 (segment (start 16.51 14.812) (end 16.51 19.05) (width 0.38) (layer "B.Cu") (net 2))
 (segment (start 7.95606 6.35) (end 6.985 7.32106) (width 0.38) (layer "B.Cu") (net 2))
 (segment (start 8.718005 19.939) (end 8.718005 24.429009) (width 0.38) (layer "B.Cu") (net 2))
 (segment (start 8.763 14.351) (end 8.763 12.7) (width 0.38) (layer "B.Cu") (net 2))
 (segment (start 11.218492 24.606473) (end 11.218492 24.595508) (width 0.38) (layer "B.Cu") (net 2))
 (segment (start 16.51 8.89) (end 16.51 13.128) (width 0.38) (layer "B.Cu") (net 2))
 (segment (start 2.794 13.65) (end 2.794 12.446) (width 0.38) (layer "B.Cu") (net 2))
 (segment (start 8.763 12.7) (end 9.537 11.926) (width 0.38) (layer "B.Cu") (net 2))
 (segment (start 8.718005 24.429009) (end 8.636 24.511014) (width 0.38) (layer "B.Cu") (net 2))
 (segment (start 3.556 6.151259) (end 3.556 9.906) (width 0.38) (layer "B.Cu") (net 2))
 (segment (start 8.636 24.511014) (end 4.191014 24.511014) (width 0.38) (layer "B.Cu") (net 2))
 (segment (start 2.794 12.446) (end 3.556 11.684) (width 0.38) (layer "B.Cu") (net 2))
 (segment (start 3.556 11.684) (end 3.556 9.906) (width 0.38) (layer "B.Cu") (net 2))
 (segment (start 13.589 22.225) (end 13.589 21.971) (width 0.38) (layer "B.Cu") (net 2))
 (segment (start 9.537 11.926) (end 9.537 10.922) (width 0.38) (layer "B.Cu") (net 2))
 (segment (start 6.985 7.32106) (end 6.985 7.747) (width 0.38) (layer "B.Cu") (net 2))
 (segment (start 2.794 17.526) (end 2.794 13.65) (width 0.38) (layer "B.Cu") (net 2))
 (segment (start 11.218492 24.595508) (end 13.589 22.225) (width 0.38) (layer "B.Cu") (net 2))
 (segment (start 15.668 13.97) (end 13.97 13.97) (width 0.38) (layer "B.Cu") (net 2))
 (segment (start 7.59 26.632) (end 7.148 26.19) (width 0.38) (layer "F.Cu") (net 4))
 (segment (start 5.258 29.083) (end 4.199 28.024) (width 0.38) (layer "F.Cu") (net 4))
 (segment (start 7.59 27.622) (end 7.59 26.632) (width 0.38) (layer "F.Cu") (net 4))
 (segment (start 7.148 26.19) (end 6.417 26.19) (width 0.38) (layer "F.Cu") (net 4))
 (segment (start 6.417 28.09) (end 7.122 28.09) (width 0.38) (layer "F.Cu") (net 4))
 (segment (start 15.24 27.94) (end 14.097 29.083) (width 0.38) (layer "F.Cu") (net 4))
 (segment (start 4.199 28.024) (end 3.272006 28.024) (width 0.38) (layer "F.Cu") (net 4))
 (segment (start 7.122 28.09) (end 7.59 27.622) (width 0.38) (layer "F.Cu") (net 4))
 (segment (start 4.199 28.024) (end 6.351 28.024) (width 0.38) (layer "F.Cu") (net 4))
 (segment (start 14.097 29.083) (end 5.258 29.083) (width 0.38) (layer "F.Cu") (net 4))
 (via (at 3.272006 28.024) (size 0.8) (drill 0.4) (layers "F.Cu" "B.Cu") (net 4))
 (segment (start 2.086006 29.21) (end 3.272006 28.024) (width 0.38) (layer "B.Cu") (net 4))
 (segment (start -1.27 1.27) (end -1.27 28.448) (width 0.38) (layer "B.Cu") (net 4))
 (segment (start 0 0) (end -1.27 1.27) (width 0.38) (layer "B.Cu") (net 4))
 (segment (start -1.27 28.448) (end -0.508 29.21) (width 0.38) (layer "B.Cu") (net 4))
 (segment (start -0.508 29.21) (end 2.086006 29.21) (width 0.38) (layer "B.Cu") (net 4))
 (segment (start 14.097 11.811) (end 14.097 11.303) (width 0.2) (layer "F.Cu") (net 19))
 (segment (start 12.713 12.431) (end 13.477 12.431) (width 0.2) (layer "F.Cu") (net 19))
 (segment (start 13.477 12.431) (end 14.097 11.811) (width 0.2) (layer "F.Cu") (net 19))
 (segment (start 14.097 11.303) (end 15.24 10.16) (width 0.2) (layer "F.Cu") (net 19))
 (segment (start 2.54 12.7) (end 3.703 12.7) (width 0.2) (layer "F.Cu") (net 7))
 (segment (start 0 10.16) (end 2.54 12.7) (width 0.2) (layer "F.Cu") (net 7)))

